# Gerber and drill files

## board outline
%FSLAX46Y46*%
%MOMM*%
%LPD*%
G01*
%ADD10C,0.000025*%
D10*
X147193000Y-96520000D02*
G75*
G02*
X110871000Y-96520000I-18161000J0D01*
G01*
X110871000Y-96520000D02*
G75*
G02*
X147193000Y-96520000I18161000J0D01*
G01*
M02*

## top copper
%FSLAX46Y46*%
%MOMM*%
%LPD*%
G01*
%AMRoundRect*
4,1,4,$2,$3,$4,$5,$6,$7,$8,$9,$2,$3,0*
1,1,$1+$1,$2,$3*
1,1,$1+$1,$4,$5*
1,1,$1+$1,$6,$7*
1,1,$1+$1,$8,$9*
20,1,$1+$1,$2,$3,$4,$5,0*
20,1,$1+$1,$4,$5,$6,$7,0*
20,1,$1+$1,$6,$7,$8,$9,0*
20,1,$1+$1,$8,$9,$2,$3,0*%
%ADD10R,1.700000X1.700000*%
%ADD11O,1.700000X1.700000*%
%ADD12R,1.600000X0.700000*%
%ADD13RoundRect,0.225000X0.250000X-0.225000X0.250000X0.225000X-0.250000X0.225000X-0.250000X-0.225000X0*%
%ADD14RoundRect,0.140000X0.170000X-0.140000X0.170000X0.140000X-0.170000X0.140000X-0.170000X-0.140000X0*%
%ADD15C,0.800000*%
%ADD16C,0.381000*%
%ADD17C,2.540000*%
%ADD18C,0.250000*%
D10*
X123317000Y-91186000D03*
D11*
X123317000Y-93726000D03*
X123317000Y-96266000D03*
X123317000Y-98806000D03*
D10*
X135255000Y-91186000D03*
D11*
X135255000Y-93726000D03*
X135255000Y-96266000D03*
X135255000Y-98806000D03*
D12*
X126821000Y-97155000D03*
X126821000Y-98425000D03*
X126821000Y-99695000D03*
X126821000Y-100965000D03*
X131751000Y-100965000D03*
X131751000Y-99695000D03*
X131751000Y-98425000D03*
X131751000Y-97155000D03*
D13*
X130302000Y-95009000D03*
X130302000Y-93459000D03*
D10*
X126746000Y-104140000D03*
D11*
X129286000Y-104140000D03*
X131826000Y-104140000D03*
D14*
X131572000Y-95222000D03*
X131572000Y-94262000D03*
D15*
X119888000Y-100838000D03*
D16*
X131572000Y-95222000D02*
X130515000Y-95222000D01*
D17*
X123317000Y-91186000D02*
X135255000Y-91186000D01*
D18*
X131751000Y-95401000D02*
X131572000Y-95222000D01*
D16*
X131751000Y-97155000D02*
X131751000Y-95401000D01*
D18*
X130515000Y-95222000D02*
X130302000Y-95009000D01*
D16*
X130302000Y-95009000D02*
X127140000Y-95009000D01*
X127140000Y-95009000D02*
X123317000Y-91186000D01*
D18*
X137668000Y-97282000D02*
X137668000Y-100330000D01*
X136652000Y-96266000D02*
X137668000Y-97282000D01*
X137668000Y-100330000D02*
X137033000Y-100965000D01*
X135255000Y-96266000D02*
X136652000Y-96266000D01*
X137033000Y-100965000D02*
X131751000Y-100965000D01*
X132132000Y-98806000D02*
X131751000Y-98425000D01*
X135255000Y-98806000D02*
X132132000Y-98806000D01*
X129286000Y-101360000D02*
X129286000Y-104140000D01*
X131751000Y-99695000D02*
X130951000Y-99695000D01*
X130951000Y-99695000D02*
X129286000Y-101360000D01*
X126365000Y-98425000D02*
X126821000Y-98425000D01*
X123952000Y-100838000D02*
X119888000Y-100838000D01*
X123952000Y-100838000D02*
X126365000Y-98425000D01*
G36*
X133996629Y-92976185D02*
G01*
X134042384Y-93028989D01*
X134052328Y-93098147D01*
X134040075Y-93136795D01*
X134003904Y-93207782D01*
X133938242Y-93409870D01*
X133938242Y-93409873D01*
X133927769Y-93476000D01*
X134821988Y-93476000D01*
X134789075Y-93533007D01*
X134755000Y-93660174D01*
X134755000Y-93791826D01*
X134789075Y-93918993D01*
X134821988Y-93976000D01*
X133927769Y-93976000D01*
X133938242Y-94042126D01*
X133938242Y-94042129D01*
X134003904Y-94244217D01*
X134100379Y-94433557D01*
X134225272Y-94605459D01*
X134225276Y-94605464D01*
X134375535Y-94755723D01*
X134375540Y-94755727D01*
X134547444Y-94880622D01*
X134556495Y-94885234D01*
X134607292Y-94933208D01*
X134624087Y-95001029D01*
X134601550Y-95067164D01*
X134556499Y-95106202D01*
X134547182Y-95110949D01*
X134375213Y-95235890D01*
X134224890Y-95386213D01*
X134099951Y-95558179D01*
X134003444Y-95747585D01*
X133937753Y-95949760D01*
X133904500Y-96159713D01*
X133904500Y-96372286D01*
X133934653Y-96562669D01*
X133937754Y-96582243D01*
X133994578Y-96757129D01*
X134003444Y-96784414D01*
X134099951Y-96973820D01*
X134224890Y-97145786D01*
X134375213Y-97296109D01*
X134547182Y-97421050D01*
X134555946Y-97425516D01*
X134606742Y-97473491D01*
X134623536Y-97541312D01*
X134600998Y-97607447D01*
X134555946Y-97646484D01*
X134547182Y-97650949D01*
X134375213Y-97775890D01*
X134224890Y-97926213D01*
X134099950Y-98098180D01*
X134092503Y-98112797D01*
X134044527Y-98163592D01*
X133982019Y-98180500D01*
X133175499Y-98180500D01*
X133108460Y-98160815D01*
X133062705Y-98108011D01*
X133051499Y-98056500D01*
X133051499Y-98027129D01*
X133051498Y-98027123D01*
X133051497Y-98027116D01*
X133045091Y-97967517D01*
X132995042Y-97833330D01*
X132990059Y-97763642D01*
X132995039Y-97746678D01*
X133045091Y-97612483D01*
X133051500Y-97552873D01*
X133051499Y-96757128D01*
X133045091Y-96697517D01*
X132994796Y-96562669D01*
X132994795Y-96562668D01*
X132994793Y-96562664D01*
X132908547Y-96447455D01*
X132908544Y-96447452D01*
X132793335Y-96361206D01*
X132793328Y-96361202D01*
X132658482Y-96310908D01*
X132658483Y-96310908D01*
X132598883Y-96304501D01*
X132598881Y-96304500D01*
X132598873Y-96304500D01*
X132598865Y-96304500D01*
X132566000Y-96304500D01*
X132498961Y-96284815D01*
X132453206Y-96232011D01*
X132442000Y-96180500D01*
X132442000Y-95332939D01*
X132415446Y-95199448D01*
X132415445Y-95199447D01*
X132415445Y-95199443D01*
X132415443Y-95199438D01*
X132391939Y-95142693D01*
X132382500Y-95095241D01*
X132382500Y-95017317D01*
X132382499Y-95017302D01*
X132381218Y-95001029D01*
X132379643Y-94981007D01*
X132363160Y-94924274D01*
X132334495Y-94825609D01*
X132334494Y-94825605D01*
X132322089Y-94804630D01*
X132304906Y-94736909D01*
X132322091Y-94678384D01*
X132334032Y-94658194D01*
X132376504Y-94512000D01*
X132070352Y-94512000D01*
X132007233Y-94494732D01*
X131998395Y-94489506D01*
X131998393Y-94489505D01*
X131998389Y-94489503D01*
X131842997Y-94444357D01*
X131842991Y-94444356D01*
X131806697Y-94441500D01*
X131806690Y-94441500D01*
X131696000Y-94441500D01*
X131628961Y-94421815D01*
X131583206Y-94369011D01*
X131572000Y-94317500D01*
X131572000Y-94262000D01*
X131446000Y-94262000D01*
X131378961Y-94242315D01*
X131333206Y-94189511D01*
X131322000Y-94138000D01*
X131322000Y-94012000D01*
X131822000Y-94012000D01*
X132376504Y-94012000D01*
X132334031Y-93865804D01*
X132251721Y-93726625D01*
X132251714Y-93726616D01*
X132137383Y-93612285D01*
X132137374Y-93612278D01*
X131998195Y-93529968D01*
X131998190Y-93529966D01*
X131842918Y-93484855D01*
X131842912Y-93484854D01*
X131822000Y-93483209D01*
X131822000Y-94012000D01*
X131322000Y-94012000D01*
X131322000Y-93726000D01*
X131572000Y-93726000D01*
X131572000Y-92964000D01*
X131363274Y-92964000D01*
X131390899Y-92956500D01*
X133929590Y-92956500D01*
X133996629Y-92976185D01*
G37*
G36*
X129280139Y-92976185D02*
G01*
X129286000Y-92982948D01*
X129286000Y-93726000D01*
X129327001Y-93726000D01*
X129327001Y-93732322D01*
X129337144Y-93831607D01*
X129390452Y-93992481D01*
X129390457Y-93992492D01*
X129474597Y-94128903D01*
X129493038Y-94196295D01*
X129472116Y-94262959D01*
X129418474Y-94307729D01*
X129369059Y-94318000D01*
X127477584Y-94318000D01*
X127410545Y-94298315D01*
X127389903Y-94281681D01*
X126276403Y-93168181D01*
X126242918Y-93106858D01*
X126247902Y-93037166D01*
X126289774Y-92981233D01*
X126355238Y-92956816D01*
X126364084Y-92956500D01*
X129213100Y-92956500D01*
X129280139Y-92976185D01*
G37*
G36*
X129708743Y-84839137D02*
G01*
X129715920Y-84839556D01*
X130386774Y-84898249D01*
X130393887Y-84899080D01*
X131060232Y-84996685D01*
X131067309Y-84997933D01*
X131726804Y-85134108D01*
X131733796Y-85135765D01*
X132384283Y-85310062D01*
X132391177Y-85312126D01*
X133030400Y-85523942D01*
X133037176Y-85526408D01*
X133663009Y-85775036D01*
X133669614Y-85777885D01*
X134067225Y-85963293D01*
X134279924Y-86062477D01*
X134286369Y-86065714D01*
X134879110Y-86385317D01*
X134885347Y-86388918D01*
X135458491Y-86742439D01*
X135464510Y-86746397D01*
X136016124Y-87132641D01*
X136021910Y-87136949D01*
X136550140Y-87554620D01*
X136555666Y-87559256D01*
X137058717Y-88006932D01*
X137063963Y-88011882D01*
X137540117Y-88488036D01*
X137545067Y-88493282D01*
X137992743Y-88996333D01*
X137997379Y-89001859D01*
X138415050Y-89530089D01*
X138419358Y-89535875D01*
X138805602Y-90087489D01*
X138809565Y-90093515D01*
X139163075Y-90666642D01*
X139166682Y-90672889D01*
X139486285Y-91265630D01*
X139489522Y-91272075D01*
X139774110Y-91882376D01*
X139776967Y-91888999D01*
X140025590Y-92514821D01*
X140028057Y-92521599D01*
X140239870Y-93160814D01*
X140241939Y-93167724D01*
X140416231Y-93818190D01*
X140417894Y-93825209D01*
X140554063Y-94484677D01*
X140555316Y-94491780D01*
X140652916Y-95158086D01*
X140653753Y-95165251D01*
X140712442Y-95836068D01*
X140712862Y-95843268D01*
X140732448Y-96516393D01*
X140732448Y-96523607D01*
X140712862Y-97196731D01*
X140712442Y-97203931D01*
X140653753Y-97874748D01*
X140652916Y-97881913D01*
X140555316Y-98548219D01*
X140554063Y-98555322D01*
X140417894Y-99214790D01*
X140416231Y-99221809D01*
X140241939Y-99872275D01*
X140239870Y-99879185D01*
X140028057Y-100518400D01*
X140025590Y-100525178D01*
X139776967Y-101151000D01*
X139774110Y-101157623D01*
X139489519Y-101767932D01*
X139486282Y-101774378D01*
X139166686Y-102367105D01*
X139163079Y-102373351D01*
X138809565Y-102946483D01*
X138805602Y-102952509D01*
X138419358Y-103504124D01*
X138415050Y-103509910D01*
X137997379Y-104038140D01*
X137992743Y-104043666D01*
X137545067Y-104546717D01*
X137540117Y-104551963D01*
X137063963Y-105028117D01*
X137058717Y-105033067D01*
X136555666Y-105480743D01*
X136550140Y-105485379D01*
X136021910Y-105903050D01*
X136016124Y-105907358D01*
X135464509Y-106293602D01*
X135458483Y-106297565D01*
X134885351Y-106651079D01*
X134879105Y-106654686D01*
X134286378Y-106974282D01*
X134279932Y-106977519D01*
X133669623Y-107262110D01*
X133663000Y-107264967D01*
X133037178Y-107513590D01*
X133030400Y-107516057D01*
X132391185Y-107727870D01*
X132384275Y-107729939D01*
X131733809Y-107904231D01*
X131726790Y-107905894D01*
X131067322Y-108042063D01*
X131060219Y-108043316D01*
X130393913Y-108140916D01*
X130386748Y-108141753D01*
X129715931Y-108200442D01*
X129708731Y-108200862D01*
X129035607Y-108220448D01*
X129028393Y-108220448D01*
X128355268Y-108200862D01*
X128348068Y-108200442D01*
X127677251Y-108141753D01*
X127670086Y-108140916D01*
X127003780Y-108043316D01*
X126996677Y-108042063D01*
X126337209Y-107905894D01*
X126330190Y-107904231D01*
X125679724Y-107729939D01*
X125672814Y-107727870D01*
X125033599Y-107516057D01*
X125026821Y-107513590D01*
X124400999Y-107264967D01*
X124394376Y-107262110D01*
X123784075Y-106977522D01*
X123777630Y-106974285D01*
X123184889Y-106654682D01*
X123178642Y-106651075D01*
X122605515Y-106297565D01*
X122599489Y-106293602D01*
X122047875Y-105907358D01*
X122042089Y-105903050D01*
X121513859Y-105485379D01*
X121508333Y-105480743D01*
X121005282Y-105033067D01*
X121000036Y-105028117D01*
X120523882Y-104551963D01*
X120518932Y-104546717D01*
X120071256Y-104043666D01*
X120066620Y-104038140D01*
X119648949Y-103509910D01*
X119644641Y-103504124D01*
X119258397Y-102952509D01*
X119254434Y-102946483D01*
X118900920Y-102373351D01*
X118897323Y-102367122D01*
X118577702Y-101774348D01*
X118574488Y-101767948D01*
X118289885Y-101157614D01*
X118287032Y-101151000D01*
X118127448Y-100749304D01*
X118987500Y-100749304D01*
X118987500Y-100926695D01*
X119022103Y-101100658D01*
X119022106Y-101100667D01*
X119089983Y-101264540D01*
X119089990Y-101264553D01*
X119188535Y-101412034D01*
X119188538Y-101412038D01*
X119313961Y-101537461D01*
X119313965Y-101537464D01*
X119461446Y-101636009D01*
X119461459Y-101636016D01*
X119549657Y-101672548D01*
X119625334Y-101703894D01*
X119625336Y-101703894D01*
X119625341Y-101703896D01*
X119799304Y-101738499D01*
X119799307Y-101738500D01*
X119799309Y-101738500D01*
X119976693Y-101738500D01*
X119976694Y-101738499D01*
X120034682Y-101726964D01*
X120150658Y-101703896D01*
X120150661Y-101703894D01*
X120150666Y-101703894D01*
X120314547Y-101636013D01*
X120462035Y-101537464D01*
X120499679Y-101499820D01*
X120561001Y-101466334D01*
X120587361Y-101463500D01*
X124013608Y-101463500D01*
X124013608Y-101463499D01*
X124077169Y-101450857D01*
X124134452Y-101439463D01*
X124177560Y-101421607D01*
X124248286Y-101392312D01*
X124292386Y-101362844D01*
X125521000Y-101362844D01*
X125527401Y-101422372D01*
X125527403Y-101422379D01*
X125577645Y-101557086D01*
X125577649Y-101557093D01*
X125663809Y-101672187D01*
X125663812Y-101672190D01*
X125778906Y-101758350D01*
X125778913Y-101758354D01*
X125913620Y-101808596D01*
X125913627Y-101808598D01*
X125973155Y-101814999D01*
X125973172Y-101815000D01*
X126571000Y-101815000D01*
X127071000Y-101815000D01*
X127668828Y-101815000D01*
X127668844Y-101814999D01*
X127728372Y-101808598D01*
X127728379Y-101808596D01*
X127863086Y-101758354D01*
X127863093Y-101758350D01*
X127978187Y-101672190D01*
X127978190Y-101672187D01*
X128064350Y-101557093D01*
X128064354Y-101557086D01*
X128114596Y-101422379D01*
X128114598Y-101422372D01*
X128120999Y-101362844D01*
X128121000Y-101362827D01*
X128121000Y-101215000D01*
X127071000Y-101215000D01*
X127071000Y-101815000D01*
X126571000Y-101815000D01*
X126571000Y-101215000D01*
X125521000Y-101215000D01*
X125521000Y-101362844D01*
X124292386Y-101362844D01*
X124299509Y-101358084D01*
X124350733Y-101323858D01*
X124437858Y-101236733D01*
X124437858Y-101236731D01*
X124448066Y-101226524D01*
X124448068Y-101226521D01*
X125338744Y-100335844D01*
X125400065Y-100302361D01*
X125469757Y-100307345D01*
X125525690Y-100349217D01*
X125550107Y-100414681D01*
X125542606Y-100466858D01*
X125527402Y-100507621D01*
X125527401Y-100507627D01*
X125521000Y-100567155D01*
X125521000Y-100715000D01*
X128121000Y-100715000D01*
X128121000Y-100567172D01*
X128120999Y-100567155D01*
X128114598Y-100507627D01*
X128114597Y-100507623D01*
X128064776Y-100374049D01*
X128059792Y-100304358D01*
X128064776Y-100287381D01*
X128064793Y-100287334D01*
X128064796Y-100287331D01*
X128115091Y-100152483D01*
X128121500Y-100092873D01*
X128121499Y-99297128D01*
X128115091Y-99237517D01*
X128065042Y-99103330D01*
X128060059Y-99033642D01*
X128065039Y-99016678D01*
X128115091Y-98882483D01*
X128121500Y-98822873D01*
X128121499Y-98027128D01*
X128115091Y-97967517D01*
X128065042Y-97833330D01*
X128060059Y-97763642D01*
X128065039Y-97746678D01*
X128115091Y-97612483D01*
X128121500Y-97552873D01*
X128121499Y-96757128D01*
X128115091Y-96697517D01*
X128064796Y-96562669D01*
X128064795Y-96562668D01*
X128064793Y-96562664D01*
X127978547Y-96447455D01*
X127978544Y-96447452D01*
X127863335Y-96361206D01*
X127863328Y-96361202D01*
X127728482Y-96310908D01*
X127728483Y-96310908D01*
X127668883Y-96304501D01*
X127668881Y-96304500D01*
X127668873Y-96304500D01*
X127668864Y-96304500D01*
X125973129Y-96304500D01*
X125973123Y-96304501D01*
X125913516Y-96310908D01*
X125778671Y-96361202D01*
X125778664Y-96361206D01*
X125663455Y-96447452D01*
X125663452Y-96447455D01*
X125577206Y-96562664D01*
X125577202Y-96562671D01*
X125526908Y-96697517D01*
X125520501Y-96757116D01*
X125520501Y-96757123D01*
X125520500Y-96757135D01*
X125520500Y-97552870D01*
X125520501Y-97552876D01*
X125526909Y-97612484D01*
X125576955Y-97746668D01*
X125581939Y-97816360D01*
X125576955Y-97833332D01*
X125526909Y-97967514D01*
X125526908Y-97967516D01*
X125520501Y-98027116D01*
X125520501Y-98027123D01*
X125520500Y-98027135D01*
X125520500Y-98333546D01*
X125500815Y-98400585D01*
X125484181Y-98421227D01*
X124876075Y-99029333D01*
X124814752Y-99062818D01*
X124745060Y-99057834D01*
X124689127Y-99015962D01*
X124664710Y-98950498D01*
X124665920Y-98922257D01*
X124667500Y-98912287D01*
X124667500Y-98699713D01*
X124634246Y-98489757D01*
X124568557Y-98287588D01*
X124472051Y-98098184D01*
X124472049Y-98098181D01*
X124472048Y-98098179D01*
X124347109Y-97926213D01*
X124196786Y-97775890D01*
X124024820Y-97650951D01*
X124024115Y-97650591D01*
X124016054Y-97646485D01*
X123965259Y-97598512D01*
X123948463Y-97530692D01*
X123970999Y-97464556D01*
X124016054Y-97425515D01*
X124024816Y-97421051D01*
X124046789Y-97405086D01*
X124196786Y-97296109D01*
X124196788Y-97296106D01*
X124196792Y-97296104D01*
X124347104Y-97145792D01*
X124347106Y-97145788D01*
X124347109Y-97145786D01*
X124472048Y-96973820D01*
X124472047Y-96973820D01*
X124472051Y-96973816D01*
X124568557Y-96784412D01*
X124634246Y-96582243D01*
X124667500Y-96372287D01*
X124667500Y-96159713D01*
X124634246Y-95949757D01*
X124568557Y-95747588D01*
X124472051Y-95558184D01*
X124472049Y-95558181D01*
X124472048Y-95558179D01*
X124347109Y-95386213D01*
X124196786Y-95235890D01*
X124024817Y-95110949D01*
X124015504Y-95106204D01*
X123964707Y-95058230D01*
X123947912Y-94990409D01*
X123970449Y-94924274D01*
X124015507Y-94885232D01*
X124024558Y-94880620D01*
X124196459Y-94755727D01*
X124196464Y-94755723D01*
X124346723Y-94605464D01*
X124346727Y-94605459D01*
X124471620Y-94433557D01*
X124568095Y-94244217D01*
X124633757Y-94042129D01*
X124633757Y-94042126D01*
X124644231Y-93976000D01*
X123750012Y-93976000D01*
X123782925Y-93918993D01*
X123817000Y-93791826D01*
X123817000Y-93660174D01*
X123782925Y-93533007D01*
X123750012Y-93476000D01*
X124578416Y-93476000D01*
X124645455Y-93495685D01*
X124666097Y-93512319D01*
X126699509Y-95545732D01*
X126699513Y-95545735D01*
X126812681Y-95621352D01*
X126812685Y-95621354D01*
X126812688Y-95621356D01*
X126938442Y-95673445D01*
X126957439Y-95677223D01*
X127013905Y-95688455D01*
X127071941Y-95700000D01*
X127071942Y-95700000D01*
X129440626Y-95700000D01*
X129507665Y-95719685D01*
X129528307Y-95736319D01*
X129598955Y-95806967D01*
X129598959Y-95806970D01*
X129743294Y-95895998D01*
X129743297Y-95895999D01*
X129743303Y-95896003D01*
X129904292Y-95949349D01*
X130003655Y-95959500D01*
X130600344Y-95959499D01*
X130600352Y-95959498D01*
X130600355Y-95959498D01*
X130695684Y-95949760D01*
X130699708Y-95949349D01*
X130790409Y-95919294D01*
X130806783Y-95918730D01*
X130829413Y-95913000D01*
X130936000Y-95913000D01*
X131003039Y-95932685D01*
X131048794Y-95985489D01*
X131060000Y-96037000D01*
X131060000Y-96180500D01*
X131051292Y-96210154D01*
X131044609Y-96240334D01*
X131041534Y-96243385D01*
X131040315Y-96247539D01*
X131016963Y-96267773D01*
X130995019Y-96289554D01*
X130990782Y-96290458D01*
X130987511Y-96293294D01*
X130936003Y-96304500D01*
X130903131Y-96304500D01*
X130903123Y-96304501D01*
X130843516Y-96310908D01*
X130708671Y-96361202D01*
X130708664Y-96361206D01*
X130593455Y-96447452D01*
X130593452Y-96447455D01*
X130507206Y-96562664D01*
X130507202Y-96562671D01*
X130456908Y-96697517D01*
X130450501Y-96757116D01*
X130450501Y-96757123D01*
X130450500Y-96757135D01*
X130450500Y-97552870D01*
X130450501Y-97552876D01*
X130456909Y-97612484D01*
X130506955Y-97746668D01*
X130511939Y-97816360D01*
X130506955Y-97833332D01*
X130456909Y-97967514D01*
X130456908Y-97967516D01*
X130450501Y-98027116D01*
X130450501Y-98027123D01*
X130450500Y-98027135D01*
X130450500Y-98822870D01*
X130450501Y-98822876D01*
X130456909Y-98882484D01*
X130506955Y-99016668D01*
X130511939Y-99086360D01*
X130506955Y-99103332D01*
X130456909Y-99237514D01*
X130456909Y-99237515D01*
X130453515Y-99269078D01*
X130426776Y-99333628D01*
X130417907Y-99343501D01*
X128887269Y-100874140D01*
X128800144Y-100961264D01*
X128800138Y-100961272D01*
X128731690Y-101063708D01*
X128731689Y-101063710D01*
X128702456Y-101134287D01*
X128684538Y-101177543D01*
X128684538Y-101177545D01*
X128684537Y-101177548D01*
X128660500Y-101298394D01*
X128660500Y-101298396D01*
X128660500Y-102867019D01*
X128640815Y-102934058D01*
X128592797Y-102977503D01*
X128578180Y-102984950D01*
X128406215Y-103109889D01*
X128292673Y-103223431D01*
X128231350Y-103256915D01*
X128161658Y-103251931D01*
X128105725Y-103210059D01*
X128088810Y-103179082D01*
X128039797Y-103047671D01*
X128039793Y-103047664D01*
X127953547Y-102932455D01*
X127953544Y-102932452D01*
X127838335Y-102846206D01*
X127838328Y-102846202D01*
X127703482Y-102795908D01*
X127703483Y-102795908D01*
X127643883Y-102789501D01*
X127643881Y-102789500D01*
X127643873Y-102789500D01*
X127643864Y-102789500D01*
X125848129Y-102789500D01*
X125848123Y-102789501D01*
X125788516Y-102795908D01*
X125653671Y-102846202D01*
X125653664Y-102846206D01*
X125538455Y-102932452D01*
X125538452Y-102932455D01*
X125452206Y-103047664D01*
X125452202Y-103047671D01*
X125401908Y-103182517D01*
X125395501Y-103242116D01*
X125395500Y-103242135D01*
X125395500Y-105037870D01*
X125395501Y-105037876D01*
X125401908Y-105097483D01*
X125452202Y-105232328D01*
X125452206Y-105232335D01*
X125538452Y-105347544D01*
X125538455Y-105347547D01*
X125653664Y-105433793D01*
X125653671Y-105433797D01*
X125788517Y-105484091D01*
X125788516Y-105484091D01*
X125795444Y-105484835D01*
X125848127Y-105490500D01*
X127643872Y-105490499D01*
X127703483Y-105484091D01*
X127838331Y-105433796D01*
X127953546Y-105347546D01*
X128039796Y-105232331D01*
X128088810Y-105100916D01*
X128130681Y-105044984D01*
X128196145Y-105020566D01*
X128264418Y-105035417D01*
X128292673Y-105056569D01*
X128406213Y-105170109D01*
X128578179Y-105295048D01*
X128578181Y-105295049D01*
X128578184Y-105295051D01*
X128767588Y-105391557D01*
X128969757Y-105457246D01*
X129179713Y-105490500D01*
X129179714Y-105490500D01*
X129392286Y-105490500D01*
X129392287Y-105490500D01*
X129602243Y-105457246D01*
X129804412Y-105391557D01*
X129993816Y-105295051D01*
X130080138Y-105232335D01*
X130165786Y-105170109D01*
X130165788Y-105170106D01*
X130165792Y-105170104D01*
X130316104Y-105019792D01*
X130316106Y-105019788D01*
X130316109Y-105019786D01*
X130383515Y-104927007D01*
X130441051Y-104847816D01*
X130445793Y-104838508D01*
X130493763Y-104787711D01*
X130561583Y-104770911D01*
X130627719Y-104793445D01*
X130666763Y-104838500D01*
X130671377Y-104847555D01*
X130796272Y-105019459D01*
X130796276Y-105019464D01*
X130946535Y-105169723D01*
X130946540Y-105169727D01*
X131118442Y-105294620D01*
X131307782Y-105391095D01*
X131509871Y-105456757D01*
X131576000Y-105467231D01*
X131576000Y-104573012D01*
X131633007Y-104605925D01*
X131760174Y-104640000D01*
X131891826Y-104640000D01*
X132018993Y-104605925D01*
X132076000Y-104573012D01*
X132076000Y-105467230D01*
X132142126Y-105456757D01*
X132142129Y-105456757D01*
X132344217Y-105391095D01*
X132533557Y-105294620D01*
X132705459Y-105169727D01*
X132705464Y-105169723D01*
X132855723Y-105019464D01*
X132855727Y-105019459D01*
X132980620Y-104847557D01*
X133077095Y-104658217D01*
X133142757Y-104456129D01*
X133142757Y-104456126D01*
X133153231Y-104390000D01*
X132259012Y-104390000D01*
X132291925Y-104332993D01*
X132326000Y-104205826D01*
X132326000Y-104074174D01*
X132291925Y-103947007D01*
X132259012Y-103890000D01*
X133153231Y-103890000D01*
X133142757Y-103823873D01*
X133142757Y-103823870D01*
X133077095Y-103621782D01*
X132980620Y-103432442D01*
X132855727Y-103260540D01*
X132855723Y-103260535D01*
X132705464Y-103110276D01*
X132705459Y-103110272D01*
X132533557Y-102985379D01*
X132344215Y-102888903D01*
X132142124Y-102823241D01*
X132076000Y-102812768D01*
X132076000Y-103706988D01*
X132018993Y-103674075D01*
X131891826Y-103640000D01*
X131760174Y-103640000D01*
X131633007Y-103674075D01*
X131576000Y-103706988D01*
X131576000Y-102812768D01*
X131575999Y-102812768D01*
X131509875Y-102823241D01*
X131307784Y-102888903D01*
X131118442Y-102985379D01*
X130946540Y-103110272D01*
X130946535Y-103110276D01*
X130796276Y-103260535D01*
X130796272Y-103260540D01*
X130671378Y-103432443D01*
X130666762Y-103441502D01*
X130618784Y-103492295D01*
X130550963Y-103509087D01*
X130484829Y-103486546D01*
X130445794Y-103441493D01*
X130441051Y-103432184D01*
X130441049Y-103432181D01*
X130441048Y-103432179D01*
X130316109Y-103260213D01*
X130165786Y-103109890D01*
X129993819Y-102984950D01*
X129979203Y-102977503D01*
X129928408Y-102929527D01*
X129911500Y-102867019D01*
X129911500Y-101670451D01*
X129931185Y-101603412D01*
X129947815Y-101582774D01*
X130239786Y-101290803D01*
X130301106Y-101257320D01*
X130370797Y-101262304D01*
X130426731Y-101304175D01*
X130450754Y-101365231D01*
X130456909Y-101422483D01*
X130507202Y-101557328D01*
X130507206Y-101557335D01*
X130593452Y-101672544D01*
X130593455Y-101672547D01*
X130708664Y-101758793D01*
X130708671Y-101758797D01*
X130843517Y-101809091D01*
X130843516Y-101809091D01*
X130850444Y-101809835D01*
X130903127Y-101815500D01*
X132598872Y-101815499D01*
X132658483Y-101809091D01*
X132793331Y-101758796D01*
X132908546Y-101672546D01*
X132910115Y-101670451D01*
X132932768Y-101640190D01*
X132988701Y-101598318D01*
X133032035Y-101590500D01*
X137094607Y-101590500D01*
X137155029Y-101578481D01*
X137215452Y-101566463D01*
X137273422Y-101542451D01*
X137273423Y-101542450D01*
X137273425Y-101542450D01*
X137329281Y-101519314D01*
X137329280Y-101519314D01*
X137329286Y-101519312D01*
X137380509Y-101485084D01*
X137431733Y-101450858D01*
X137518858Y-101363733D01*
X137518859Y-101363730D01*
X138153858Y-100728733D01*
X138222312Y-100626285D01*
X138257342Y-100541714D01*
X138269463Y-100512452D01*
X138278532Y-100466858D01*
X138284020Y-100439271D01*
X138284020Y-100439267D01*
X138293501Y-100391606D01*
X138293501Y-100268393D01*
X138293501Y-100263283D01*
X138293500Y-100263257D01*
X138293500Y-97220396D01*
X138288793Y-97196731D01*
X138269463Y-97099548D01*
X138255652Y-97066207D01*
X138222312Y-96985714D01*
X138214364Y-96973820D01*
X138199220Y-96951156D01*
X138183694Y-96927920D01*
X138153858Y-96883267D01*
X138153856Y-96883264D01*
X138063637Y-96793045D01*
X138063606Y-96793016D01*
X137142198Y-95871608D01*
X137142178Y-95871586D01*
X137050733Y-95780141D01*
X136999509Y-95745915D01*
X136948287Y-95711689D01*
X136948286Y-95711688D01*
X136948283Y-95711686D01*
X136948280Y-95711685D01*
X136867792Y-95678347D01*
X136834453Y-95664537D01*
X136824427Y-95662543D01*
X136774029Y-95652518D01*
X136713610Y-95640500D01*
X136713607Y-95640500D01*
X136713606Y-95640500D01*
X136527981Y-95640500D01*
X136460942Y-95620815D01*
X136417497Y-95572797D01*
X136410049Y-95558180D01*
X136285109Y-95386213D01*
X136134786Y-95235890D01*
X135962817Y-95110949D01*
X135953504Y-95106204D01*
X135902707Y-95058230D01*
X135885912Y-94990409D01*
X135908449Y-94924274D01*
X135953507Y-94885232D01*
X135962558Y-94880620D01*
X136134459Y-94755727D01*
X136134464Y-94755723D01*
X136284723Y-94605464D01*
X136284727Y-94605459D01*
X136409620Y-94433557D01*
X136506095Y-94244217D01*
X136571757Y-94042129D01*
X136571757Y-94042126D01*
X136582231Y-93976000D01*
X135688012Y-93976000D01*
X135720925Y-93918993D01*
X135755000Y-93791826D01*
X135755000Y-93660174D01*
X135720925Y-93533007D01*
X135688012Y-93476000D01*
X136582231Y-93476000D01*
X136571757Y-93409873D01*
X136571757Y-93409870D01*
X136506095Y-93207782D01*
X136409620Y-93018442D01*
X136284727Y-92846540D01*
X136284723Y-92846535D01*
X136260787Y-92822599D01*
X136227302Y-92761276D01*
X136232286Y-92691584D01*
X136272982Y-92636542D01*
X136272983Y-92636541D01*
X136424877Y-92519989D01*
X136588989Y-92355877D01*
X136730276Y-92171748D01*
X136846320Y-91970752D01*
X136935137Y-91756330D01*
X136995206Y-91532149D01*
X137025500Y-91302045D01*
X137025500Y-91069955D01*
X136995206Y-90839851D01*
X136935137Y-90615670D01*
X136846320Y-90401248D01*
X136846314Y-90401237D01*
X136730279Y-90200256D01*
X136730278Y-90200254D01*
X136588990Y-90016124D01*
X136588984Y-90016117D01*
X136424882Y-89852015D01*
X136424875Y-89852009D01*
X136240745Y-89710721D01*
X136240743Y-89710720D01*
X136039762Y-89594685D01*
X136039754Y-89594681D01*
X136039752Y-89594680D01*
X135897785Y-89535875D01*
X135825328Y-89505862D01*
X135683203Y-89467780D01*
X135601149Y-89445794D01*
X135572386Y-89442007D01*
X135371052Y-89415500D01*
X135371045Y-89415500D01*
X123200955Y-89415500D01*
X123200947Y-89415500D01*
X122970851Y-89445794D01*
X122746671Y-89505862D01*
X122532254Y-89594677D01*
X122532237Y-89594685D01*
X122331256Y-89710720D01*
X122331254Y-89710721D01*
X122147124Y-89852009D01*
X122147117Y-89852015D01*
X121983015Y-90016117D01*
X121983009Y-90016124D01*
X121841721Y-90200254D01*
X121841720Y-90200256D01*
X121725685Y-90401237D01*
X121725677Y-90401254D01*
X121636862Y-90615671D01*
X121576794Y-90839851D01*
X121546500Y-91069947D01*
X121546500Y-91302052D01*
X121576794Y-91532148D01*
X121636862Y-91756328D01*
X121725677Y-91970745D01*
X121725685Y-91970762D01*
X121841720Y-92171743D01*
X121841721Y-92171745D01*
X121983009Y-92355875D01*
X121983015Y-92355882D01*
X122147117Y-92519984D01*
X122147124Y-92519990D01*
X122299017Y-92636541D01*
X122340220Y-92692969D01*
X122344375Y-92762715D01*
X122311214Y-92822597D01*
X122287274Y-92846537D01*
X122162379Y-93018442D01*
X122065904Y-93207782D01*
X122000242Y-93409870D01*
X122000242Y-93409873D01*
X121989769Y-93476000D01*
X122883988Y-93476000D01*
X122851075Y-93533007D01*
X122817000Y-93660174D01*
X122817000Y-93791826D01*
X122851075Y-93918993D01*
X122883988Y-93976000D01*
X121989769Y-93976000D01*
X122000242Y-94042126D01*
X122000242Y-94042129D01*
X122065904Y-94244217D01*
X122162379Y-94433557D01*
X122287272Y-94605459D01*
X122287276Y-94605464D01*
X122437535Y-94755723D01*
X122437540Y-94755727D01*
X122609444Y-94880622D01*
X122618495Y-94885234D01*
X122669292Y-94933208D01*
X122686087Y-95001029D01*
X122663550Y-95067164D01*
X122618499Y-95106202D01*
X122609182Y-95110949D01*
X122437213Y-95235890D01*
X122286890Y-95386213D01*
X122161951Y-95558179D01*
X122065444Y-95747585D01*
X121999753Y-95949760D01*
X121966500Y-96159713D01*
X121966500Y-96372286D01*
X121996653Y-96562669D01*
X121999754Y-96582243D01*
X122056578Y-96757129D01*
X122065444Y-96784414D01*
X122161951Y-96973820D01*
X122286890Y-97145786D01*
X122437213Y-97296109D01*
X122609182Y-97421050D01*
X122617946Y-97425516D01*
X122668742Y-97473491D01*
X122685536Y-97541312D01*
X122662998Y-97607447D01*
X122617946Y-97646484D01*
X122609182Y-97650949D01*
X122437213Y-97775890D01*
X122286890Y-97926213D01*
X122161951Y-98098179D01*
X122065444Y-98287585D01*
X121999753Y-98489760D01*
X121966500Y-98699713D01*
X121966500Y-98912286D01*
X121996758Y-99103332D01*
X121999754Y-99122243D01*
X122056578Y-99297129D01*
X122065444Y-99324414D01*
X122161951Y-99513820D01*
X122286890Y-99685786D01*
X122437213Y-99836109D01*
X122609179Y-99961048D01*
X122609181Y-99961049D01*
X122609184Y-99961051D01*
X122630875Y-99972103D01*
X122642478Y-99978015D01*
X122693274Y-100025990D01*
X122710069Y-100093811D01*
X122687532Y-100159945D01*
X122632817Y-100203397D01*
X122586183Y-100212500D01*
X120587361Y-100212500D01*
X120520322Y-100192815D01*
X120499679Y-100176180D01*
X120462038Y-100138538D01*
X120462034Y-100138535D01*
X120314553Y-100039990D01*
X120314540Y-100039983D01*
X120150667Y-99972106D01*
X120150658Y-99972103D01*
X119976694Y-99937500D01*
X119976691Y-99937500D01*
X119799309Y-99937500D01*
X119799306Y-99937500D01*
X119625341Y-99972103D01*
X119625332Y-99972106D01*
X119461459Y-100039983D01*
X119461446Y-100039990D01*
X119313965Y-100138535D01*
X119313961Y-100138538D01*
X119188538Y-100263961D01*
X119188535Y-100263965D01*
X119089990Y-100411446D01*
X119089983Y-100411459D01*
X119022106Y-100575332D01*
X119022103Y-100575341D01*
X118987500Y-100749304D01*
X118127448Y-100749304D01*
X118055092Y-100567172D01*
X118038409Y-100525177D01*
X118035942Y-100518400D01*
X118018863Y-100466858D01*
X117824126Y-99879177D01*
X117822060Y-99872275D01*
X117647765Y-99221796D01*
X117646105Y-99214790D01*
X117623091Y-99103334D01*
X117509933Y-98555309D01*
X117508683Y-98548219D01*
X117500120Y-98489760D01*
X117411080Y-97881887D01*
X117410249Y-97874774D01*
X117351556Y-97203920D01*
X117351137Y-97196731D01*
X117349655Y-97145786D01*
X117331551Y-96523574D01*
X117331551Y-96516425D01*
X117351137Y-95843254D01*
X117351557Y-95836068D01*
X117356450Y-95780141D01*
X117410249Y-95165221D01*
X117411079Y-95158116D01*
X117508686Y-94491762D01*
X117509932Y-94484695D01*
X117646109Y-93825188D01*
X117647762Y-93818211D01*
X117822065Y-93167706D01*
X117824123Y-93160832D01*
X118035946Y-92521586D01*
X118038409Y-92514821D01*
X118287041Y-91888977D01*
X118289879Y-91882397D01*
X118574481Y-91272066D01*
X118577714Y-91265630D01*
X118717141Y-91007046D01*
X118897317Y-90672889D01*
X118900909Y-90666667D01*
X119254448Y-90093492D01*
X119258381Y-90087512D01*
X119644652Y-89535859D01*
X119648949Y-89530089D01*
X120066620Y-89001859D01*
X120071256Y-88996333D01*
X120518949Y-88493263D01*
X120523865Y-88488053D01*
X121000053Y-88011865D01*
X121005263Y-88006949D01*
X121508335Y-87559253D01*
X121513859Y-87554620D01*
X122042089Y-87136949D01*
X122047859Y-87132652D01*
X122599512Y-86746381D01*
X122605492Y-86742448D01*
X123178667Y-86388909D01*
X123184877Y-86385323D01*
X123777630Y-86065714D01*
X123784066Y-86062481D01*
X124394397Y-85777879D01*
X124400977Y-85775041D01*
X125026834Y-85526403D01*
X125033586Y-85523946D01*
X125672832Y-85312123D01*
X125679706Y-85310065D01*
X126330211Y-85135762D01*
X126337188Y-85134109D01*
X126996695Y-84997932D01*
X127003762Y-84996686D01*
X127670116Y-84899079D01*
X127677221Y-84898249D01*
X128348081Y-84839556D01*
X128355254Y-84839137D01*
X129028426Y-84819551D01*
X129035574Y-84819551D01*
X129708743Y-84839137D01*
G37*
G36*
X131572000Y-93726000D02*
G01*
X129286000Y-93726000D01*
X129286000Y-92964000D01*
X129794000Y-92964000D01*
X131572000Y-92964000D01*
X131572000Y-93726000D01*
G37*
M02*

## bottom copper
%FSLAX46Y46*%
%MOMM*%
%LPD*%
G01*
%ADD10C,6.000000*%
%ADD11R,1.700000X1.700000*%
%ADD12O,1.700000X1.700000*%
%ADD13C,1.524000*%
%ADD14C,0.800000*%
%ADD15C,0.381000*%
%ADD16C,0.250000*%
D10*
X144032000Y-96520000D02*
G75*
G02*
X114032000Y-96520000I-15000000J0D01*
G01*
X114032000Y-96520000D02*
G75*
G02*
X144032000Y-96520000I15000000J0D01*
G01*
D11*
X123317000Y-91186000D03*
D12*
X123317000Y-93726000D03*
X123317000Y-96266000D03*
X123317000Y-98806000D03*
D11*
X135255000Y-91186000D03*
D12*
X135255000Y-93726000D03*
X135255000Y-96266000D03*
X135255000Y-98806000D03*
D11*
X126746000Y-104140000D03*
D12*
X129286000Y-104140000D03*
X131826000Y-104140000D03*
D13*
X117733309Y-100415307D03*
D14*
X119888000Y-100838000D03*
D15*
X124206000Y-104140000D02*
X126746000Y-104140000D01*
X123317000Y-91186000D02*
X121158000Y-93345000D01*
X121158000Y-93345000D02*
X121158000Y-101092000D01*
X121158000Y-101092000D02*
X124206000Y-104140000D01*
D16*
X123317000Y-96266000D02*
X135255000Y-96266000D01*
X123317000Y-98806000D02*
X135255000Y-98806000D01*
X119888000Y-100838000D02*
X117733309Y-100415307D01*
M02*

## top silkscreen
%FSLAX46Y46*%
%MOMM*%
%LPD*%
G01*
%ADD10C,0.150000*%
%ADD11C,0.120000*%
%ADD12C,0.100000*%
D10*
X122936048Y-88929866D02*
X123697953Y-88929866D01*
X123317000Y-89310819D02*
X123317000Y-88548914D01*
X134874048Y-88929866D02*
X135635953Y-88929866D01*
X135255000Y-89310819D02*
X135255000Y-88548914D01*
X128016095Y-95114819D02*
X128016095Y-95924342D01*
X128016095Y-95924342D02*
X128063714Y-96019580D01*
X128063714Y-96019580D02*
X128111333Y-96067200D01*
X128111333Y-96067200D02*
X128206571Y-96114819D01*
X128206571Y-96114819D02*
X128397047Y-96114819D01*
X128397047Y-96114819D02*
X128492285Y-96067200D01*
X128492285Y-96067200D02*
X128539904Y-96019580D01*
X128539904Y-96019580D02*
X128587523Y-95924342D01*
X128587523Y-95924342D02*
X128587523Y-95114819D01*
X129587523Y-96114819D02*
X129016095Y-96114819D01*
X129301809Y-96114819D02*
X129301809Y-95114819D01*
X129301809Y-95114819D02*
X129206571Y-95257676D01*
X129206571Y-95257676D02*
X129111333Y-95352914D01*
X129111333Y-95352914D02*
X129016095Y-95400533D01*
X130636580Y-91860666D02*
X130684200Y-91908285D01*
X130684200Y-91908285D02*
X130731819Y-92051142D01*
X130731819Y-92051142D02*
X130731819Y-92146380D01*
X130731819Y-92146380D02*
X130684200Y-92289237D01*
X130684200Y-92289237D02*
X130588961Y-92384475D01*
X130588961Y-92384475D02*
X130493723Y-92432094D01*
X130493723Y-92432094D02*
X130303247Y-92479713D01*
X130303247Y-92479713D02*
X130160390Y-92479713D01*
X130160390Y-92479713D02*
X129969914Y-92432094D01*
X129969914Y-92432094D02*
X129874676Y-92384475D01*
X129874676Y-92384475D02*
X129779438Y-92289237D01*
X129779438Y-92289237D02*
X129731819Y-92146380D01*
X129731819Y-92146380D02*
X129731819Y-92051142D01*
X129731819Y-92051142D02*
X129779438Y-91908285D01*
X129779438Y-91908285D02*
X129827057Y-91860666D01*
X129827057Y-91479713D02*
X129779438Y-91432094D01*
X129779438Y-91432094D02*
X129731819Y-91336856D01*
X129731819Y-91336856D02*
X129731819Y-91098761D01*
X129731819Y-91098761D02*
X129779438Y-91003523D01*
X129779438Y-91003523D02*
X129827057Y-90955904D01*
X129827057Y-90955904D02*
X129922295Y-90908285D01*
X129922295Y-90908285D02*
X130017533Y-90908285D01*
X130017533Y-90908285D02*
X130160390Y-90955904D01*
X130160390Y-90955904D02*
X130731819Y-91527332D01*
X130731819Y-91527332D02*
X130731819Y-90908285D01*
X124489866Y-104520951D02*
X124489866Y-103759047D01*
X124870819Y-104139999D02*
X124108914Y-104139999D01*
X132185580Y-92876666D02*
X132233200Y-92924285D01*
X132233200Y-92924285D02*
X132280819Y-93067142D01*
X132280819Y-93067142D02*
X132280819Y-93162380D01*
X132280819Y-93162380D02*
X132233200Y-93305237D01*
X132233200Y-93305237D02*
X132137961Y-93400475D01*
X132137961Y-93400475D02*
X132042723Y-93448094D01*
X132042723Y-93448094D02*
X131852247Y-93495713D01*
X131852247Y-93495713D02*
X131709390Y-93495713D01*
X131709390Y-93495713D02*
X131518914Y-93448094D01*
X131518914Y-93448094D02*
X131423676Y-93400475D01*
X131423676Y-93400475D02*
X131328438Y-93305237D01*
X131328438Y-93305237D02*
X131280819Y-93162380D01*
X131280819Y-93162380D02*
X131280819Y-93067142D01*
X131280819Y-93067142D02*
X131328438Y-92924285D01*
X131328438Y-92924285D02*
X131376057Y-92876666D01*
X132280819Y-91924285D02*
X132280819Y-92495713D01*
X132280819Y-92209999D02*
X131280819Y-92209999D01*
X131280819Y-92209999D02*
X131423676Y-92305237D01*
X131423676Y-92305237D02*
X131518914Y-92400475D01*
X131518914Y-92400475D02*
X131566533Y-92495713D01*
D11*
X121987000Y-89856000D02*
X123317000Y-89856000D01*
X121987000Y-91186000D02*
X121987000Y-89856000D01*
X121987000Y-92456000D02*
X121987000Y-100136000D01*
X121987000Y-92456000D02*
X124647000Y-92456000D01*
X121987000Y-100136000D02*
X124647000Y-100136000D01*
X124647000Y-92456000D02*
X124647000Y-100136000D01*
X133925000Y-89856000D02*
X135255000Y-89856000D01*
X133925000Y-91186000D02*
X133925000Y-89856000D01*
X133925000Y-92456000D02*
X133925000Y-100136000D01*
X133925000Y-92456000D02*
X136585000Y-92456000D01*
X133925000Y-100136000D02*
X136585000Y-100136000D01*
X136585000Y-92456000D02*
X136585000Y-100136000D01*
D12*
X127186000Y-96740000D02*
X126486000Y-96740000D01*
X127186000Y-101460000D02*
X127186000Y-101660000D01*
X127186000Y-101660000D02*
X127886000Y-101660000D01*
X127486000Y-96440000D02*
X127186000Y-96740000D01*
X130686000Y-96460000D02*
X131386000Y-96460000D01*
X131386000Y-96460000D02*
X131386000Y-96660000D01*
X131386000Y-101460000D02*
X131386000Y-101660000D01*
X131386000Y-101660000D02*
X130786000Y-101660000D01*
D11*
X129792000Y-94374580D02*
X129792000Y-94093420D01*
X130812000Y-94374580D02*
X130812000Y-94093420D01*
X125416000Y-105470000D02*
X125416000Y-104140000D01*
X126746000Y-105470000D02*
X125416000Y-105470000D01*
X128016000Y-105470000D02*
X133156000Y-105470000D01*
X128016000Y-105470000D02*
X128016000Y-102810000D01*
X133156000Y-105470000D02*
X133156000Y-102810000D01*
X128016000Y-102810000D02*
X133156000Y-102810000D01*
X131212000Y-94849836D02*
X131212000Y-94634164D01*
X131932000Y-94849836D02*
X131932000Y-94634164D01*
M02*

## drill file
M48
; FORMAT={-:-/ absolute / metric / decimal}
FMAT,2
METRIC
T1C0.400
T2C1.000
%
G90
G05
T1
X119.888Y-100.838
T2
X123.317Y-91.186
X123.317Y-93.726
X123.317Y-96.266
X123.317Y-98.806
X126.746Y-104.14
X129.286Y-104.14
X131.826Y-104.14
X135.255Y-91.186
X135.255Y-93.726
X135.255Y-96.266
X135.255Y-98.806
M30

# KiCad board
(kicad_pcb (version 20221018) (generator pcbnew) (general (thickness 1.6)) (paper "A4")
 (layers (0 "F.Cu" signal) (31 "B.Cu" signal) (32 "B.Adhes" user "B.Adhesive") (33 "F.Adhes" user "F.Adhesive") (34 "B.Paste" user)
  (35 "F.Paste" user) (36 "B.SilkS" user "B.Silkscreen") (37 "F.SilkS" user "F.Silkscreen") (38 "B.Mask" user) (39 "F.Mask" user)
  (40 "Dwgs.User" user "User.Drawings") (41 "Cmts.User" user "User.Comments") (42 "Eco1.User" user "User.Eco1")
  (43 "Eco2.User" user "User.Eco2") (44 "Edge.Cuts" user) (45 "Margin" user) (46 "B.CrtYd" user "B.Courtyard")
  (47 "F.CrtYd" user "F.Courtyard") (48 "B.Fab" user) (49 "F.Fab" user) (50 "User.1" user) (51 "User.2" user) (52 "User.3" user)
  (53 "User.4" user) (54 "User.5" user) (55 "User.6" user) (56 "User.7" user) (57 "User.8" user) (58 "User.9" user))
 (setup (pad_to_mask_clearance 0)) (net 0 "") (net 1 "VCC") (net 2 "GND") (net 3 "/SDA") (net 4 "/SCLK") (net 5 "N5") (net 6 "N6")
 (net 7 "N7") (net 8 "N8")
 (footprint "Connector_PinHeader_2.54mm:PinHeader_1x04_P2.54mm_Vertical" (layer "F.Cu") (at 123.317 91.186)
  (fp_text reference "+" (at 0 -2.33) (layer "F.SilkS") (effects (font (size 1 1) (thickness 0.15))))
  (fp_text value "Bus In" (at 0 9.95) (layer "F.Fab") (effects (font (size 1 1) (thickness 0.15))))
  (fp_line (start -1.33 -1.33) (end 0 -1.33) (stroke (width 0.12) (type solid)) (layer "F.SilkS"))
  (fp_line (start -1.33 0) (end -1.33 -1.33) (stroke (width 0.12) (type solid)) (layer "F.SilkS"))
  (fp_line (start -1.33 1.27) (end -1.33 8.95) (stroke (width 0.12) (type solid)) (layer "F.SilkS"))
  (fp_line (start -1.33 1.27) (end 1.33 1.27) (stroke (width 0.12) (type solid)) (layer "F.SilkS"))
  (fp_line (start -1.33 8.95) (end 1.33 8.95) (stroke (width 0.12) (type solid)) (layer "F.SilkS"))
  (fp_line (start 1.33 1.27) (end 1.33 8.95) (stroke (width 0.12) (type solid)) (layer "F.SilkS"))
  (pad "1" thru_hole rect (at 0 0) (size 1.7 1.7) (drill 1) (layers "*.Cu" "*.Mask") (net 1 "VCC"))
  (pad "2" thru_hole oval (at 0 2.54) (size 1.7 1.7) (drill 1) (layers "*.Cu" "*.Mask") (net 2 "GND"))
  (pad "3" thru_hole oval (at 0 5.08) (size 1.7 1.7) (drill 1) (layers "*.Cu" "*.Mask") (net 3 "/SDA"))
  (pad "4" thru_hole oval (at 0 7.62) (size 1.7 1.7) (drill 1) (layers "*.Cu" "*.Mask") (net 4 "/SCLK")))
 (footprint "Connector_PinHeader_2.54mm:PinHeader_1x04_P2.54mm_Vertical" (layer "F.Cu") (at 135.255 91.186)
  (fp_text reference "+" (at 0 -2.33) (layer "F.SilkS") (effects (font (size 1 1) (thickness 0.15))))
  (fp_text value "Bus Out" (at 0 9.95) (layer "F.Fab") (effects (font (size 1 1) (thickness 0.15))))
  (fp_line (start -1.33 -1.33) (end 0 -1.33) (stroke (width 0.12) (type solid)) (layer "F.SilkS"))
  (fp_line (start -1.33 0) (end -1.33 -1.33) (stroke (width 0.12) (type solid)) (layer "F.SilkS"))
  (fp_line (start -1.33 1.27) (end -1.33 8.95) (stroke (width 0.12) (type solid)) (layer "F.SilkS"))
  (fp_line (start -1.33 1.27) (end 1.33 1.27) (stroke (width 0.12) (type solid)) (layer "F.SilkS"))
  (fp_line (start -1.33 8.95) (end 1.33 8.95) (stroke (width 0.12) (type solid)) (layer "F.SilkS"))
  (fp_line (start 1.33 1.27) (end 1.33 8.95) (stroke (width 0.12) (type solid)) (layer "F.SilkS"))
  (pad "1" thru_hole rect (at 0 0) (size 1.7 1.7) (drill 1) (layers "*.Cu" "*.Mask") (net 1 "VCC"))
  (pad "2" thru_hole oval (at 0 2.54) (size 1.7 1.7) (drill 1) (layers "*.Cu" "*.Mask") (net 2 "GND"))
  (pad "3" thru_hole oval (at 0 5.08) (size 1.7 1.7) (drill 1) (layers "*.Cu" "*.Mask") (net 3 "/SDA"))
  (pad "4" thru_hole oval (at 0 7.62) (size 1.7 1.7) (drill 1) (layers "*.Cu" "*.Mask") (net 4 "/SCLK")))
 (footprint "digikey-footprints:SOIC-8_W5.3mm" (layer "F.Cu") (at 129.286 99.06)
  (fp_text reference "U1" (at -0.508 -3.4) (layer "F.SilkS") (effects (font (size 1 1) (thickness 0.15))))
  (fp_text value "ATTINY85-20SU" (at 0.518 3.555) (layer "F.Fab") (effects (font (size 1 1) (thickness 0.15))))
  (fp_line (start -2.1 -2.32) (end -2.8 -2.32) (stroke (width 0.1) (type solid)) (layer "F.SilkS"))
  (fp_line (start -2.1 2.4) (end -2.1 2.6) (stroke (width 0.1) (type solid)) (layer "F.SilkS"))
  (fp_line (start -2.1 2.6) (end -1.4 2.6) (stroke (width 0.1) (type solid)) (layer "F.SilkS"))
  (fp_line (start -1.8 -2.62) (end -2.1 -2.32) (stroke (width 0.1) (type solid)) (layer "F.SilkS"))
  (fp_line (start 1.4 -2.6) (end 2.1 -2.6) (stroke (width 0.1) (type solid)) (layer "F.SilkS"))
  (fp_line (start 2.1 -2.6) (end 2.1 -2.4) (stroke (width 0.1) (type solid)) (layer "F.SilkS"))
  (fp_line (start 2.1 2.4) (end 2.1 2.6) (stroke (width 0.1) (type solid)) (layer "F.SilkS"))
  (fp_line (start 2.1 2.6) (end 1.5 2.6) (stroke (width 0.1) (type solid)) (layer "F.SilkS"))
  (pad "1" smd rect (at -2.465 -1.905) (size 1.6 0.7) (layers "F.Cu" "F.Paste" "F.Mask") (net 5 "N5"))
  (pad "2" smd rect (at -2.465 -0.635) (size 1.6 0.7) (layers "F.Cu" "F.Paste" "F.Mask") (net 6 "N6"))
  (pad "3" smd rect (at -2.465 0.635) (size 1.6 0.7) (layers "F.Cu" "F.Paste" "F.Mask") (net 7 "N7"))
  (pad "4" smd rect (at -2.465 1.905) (size 1.6 0.7) (layers "F.Cu" "F.Paste" "F.Mask") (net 2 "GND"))
  (pad "5" smd rect (at 2.465 1.905) (size 1.6 0.7) (layers "F.Cu" "F.Paste" "F.Mask") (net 3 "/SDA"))
  (pad "6" smd rect (at 2.465 0.635) (size 1.6 0.7) (layers "F.Cu" "F.Paste" "F.Mask") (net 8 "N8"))
  (pad "7" smd rect (at 2.465 -0.635) (size 1.6 0.7) (layers "F.Cu" "F.Paste" "F.Mask") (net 4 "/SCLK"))
  (pad "8" smd rect (at 2.465 -1.905) (size 1.6 0.7) (layers "F.Cu" "F.Paste" "F.Mask") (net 1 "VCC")))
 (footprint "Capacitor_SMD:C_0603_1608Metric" (layer "F.Cu") (at 130.302 94.234 90)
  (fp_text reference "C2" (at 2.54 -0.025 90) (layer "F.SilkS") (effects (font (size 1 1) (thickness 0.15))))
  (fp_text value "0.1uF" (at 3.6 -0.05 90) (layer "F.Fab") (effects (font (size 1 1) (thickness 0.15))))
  (fp_line (start -0.14058 -0.51) (end 0.14058 -0.51) (stroke (width 0.12) (type solid)) (layer "F.SilkS"))
  (fp_line (start -0.14058 0.51) (end 0.14058 0.51) (stroke (width 0.12) (type solid)) (layer "F.SilkS"))
  (pad "1" smd roundrect (at -0.775 0 90) (size 0.9 0.95) (layers "F.Cu" "F.Paste" "F.Mask") (roundrect_rratio 0.25) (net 1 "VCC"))
  (pad "2" smd roundrect (at 0.775 0 90) (size 0.9 0.95) (layers "F.Cu" "F.Paste" "F.Mask") (roundrect_rratio 0.25) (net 2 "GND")))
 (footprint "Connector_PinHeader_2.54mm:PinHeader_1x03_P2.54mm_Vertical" (layer "F.Cu") (at 126.746 104.14 90)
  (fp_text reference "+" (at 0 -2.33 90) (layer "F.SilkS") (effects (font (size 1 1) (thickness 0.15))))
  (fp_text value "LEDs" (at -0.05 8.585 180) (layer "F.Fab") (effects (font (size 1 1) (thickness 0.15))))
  (fp_line (start -1.33 -1.33) (end 0 -1.33) (stroke (width 0.12) (type solid)) (layer "F.SilkS"))
  (fp_line (start -1.33 0) (end -1.33 -1.33) (stroke (width 0.12) (type solid)) (layer "F.SilkS"))
  (fp_line (start -1.33 1.27) (end -1.33 6.41) (stroke (width 0.12) (type solid)) (layer "F.SilkS"))
  (fp_line (start -1.33 1.27) (end 1.33 1.27) (stroke (width 0.12) (type solid)) (layer "F.SilkS"))
  (fp_line (start -1.33 6.41) (end 1.33 6.41) (stroke (width 0.12) (type solid)) (layer "F.SilkS"))
  (fp_line (start 1.33 1.27) (end 1.33 6.41) (stroke (width 0.12) (type solid)) (layer "F.SilkS"))
  (pad "1" thru_hole rect (at 0 0 90) (size 1.7 1.7) (drill 1) (layers "*.Cu" "*.Mask") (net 1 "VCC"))
  (pad "2" thru_hole oval (at 0 2.54 90) (size 1.7 1.7) (drill 1) (layers "*.Cu" "*.Mask") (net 8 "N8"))
  (pad "3" thru_hole oval (at 0 5.08 90) (size 1.7 1.7) (drill 1) (layers "*.Cu" "*.Mask") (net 2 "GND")))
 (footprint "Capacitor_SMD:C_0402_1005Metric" (layer "F.Cu") (at 131.572 94.742 90)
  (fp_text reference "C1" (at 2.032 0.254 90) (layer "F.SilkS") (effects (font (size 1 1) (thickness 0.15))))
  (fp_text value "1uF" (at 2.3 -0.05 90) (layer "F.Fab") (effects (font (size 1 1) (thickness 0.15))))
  (fp_line (start -0.107836 -0.36) (end 0.107836 -0.36) (stroke (width 0.12) (type solid)) (layer "F.SilkS"))
  (fp_line (start -0.107836 0.36) (end 0.107836 0.36) (stroke (width 0.12) (type solid)) (layer "F.SilkS"))
  (pad "1" smd roundrect (at -0.48 0 90) (size 0.56 0.62) (layers "F.Cu" "F.Paste" "F.Mask") (roundrect_rratio 0.25) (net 1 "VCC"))
  (pad "2" smd roundrect (at 0.48 0 90) (size 0.56 0.62) (layers "F.Cu" "F.Paste" "F.Mask") (roundrect_rratio 0.25) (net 2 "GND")))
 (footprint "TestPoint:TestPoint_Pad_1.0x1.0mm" (layer "B.Cu") (at 129.032 96.52 180)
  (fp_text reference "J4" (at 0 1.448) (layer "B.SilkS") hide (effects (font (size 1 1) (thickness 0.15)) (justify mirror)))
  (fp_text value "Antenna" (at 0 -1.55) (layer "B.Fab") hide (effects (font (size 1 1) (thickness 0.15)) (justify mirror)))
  (fp_circle (center 0 0) (end 15 0) (stroke (width 6) (type default)) (fill none) (layer "B.Cu"))
  (pad "1" smd circle (at 11.298691 -3.895307 180) (size 1.524 1.524) (layers "B.Cu" "B.Paste" "B.Mask")))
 (gr_circle (center 129.032 96.52) (end 147.193 96.52) (stroke (width 0.000025) (type default)) (fill none) (layer "Edge.Cuts"))
 (segment (start 131.572 95.222) (end 130.515 95.222) (width 0.381) (layer "F.Cu") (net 1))
 (segment (start 123.317 91.186) (end 135.255 91.186) (width 2.54) (layer "F.Cu") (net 1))
 (segment (start 131.751 95.401) (end 131.572 95.222) (width 0.25) (layer "F.Cu") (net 1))
 (segment (start 131.751 97.155) (end 131.751 95.401) (width 0.381) (layer "F.Cu") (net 1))
 (segment (start 130.515 95.222) (end 130.302 95.009) (width 0.25) (layer "F.Cu") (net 1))
 (segment (start 130.302 95.009) (end 127.14 95.009) (width 0.381) (layer "F.Cu") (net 1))
 (segment (start 127.14 95.009) (end 123.317 91.186) (width 0.381) (layer "F.Cu") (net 1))
 (segment (start 124.206 104.14) (end 126.746 104.14) (width 0.381) (layer "B.Cu") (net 1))
 (segment (start 123.317 91.186) (end 121.158 93.345) (width 0.381) (layer "B.Cu") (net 1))
 (segment (start 121.158 93.345) (end 121.158 101.092) (width 0.381) (layer "B.Cu") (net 1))
 (segment (start 121.158 101.092) (end 124.206 104.14) (width 0.381) (layer "B.Cu") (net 1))
 (segment (start 137.668 97.282) (end 137.668 100.33) (width 0.25) (layer "F.Cu") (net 3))
 (segment (start 136.652 96.266) (end 137.668 97.282) (width 0.25) (layer "F.Cu") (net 3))
 (segment (start 137.668 100.33) (end 137.033 100.965) (width 0.25) (layer "F.Cu") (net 3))
 (segment (start 135.255 96.266) (end 136.652 96.266) (width 0.25) (layer "F.Cu") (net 3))
 (segment (start 137.033 100.965) (end 131.751 100.965) (width 0.25) (layer "F.Cu") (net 3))
 (segment (start 123.317 96.266) (end 135.255 96.266) (width 0.25) (layer "B.Cu") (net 3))
 (segment (start 132.132 98.806) (end 131.751 98.425) (width 0.25) (layer "F.Cu") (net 4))
 (segment (start 135.255 98.806) (end 132.132 98.806) (width 0.25) (layer "F.Cu") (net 4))
 (segment (start 123.317 98.806) (end 135.255 98.806) (width 0.25) (layer "B.Cu") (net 4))
 (segment (start 129.286 101.36) (end 129.286 104.14) (width 0.25) (layer "F.Cu") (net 8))
 (segment (start 131.751 99.695) (end 130.951 99.695) (width 0.25) (layer "F.Cu") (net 8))
 (segment (start 130.951 99.695) (end 129.286 101.36) (width 0.25) (layer "F.Cu") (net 8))
 (segment (start 126.365 98.425) (end 126.821 98.425) (width 0.25) (layer "F.Cu") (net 6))
 (segment (start 123.952 100.838) (end 119.888 100.838) (width 0.25) (layer "F.Cu") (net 6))
 (segment (start 123.952 100.838) (end 126.365 98.425) (width 0.25) (layer "F.Cu") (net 6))
 (via (at 119.888 100.838) (size 0.8) (drill 0.4) (layers "F.Cu" "B.Cu") (free) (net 6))
 (segment (start 119.888 100.838) (end 117.733309 100.415307) (width 0.25) (layer "B.Cu") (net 6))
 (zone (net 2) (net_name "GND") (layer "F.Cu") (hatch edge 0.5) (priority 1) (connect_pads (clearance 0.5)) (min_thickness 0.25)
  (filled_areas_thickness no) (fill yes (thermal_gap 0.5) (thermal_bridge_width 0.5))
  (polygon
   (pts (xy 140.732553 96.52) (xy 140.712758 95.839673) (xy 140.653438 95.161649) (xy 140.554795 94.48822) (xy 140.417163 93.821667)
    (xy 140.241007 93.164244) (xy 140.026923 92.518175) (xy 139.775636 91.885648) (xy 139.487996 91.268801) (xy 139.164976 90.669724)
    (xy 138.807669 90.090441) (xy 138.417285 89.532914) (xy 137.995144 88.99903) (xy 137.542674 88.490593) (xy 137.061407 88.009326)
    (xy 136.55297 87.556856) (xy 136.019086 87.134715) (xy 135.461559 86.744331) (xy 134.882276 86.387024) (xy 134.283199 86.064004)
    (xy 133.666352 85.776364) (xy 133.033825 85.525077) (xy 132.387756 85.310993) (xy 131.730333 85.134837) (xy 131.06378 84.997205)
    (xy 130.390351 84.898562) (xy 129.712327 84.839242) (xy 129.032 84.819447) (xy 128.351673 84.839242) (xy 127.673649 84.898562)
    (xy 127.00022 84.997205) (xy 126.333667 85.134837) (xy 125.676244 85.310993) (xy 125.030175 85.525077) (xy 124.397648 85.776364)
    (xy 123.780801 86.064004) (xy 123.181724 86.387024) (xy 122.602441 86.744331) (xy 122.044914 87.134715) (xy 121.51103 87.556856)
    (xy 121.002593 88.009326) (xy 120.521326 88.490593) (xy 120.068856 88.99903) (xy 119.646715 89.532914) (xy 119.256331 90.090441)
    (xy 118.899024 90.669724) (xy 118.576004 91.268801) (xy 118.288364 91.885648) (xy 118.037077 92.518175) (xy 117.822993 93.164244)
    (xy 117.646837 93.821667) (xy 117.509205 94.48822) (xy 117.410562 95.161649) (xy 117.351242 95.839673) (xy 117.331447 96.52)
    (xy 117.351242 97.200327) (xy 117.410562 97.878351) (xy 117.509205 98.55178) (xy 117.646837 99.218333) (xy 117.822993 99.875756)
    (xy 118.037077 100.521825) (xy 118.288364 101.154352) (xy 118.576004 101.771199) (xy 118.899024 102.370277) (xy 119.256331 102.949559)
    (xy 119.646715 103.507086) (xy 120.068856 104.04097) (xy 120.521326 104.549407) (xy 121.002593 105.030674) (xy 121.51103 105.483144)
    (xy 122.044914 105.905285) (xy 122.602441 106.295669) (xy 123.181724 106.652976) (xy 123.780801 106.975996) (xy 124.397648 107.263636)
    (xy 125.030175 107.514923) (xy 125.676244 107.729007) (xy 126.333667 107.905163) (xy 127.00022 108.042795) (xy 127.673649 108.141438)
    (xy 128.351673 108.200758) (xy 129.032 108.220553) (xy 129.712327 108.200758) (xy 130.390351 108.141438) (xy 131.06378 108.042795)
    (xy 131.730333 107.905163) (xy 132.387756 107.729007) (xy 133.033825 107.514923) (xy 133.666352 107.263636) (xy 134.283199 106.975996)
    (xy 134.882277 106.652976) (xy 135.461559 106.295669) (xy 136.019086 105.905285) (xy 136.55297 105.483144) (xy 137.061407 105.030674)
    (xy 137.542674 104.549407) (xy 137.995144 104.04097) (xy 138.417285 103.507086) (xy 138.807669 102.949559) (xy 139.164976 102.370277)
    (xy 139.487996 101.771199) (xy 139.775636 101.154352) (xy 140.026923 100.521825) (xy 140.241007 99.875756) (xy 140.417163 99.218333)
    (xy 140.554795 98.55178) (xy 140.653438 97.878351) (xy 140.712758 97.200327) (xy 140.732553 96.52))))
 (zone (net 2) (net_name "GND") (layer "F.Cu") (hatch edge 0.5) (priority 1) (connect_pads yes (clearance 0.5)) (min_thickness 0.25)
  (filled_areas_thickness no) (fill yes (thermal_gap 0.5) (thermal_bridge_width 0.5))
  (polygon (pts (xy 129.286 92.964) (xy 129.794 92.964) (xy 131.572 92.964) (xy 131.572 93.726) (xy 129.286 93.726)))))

